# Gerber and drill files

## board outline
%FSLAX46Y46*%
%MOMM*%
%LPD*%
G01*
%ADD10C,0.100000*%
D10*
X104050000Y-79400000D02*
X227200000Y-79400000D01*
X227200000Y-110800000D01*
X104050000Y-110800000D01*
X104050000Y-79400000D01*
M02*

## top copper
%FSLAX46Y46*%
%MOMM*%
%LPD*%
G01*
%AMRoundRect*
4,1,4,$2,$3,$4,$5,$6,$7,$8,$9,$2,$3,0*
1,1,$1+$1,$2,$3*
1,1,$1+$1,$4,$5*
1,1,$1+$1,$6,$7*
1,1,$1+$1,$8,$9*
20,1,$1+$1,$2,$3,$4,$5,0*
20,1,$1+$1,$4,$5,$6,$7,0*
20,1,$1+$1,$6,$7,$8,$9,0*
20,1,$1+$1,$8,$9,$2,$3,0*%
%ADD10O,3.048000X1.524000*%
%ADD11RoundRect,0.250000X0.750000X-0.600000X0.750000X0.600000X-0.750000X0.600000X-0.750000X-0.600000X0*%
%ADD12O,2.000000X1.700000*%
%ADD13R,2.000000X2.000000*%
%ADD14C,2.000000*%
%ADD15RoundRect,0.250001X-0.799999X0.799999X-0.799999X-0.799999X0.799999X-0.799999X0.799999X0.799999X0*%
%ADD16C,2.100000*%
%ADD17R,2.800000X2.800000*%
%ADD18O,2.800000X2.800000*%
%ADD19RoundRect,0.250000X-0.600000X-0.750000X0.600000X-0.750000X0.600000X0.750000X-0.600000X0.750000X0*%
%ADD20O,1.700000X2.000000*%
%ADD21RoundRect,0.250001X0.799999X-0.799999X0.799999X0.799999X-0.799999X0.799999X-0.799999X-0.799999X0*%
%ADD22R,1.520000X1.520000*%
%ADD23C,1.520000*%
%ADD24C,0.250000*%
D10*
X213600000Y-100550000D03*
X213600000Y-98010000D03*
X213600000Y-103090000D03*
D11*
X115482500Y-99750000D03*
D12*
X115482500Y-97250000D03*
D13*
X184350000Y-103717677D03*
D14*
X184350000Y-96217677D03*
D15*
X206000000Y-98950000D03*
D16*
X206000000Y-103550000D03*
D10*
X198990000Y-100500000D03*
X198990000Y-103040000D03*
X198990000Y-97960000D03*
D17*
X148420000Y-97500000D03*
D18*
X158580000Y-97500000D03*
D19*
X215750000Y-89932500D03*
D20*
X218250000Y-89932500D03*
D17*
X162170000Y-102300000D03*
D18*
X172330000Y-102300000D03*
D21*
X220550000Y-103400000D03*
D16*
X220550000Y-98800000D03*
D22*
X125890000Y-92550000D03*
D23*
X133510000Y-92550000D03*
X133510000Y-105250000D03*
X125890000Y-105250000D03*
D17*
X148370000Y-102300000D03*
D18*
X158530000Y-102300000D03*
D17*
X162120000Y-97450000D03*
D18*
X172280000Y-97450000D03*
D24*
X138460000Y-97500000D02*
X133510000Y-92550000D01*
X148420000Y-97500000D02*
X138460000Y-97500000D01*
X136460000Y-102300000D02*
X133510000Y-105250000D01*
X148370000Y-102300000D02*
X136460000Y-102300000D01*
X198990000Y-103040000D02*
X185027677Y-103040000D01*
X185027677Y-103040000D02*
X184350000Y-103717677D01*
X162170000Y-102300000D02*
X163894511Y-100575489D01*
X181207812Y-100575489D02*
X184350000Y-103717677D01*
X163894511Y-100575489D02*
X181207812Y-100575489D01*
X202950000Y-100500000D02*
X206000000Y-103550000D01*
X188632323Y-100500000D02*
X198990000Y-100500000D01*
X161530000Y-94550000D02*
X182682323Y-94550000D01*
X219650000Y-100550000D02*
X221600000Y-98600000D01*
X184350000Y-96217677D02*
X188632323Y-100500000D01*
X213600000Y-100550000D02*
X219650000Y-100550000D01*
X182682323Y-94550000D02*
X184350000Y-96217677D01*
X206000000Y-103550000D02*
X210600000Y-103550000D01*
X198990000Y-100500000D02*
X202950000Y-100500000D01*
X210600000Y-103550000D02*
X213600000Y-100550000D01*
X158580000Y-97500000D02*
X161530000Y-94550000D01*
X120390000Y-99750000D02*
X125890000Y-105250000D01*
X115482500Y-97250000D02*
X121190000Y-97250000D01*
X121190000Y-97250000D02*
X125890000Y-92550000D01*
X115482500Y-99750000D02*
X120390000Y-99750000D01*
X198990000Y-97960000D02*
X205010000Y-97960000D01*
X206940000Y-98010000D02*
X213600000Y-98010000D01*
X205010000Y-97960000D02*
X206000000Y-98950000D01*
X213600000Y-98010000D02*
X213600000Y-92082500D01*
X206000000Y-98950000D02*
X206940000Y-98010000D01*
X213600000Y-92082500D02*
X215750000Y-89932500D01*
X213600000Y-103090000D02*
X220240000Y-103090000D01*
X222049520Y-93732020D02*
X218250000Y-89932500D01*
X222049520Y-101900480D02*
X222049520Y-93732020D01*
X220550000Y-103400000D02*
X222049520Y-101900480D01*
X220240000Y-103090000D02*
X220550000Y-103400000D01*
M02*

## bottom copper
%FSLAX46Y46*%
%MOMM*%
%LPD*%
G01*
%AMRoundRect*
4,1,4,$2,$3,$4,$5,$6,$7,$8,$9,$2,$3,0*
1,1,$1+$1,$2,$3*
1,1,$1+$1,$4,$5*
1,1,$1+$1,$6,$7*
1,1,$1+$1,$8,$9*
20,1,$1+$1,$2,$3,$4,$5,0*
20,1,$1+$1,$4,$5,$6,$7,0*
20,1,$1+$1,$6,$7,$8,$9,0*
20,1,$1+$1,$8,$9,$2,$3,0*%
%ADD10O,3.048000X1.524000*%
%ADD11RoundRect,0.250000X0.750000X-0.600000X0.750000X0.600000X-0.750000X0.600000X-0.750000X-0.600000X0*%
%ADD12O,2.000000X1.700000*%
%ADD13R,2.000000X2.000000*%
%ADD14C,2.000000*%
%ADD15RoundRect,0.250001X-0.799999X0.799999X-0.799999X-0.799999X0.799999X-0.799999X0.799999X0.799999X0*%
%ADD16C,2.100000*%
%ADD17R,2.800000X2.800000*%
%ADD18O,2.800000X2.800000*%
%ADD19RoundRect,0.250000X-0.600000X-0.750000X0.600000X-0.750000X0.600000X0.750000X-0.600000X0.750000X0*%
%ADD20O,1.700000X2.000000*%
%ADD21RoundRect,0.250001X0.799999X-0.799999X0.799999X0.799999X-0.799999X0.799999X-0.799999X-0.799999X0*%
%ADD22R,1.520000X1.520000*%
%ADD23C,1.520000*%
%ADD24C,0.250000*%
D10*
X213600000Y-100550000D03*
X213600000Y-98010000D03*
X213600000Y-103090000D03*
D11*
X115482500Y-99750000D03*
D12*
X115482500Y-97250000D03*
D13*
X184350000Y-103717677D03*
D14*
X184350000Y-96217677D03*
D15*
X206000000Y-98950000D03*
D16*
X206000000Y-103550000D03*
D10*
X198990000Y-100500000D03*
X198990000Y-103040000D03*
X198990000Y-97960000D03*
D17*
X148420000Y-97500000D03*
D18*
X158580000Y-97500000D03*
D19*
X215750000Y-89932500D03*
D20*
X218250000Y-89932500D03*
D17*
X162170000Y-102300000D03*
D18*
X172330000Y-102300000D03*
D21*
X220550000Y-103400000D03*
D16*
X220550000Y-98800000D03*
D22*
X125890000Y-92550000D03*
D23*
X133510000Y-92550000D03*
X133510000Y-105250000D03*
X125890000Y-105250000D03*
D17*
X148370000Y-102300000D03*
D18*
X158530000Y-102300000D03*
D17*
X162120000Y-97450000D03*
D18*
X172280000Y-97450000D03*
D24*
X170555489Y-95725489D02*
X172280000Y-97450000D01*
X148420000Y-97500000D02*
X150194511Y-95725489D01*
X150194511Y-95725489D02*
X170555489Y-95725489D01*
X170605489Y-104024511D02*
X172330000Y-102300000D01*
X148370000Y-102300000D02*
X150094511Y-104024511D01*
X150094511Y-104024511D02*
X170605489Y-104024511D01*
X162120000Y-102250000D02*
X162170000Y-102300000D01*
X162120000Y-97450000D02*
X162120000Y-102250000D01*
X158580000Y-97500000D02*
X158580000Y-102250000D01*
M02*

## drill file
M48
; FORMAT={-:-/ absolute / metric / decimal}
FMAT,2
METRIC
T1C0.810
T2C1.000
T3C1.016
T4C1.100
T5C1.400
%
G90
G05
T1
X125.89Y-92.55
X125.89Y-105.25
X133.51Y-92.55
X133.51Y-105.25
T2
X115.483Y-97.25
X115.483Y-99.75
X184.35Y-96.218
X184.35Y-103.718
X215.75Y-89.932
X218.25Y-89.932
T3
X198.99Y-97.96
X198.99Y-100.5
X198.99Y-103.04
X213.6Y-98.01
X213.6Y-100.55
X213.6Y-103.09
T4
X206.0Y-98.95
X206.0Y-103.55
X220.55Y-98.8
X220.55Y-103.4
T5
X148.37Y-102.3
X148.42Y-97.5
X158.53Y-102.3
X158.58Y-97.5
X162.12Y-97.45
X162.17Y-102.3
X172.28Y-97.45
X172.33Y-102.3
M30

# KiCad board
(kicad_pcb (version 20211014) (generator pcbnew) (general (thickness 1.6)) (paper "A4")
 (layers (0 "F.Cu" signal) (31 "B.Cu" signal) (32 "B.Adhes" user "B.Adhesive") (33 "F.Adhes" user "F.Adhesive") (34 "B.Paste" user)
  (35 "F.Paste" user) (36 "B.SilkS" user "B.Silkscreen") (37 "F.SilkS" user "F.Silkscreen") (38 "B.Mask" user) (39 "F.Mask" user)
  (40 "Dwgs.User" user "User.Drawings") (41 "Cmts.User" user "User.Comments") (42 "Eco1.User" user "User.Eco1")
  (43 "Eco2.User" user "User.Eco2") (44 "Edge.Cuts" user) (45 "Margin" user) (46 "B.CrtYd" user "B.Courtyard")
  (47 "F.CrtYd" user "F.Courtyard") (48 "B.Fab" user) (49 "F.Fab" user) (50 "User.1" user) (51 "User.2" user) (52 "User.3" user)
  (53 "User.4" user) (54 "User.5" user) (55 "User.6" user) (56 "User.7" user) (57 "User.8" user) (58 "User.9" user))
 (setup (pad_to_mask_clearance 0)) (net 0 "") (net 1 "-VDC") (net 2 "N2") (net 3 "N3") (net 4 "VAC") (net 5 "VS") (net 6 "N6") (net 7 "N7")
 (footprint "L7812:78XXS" (layer "F.Cu") (at 216.14 100.55 -90)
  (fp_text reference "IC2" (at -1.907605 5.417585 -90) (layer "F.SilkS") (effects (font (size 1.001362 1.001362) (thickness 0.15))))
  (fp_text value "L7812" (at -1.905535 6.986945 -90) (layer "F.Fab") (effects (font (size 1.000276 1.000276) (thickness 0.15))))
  (pad "GND" thru_hole oval locked (at 0 2.54 270) (size 1.524 3.048) (drill 1.016) (layers *.Cu *.Mask) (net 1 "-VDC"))
  (pad "IN" thru_hole oval locked (at -2.54 2.54 270) (size 1.524 3.048) (drill 1.016) (layers *.Cu *.Mask) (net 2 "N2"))
  (pad "OUT" thru_hole oval locked (at 2.54 2.54 270) (size 1.524 3.048) (drill 1.016) (layers *.Cu *.Mask) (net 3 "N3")))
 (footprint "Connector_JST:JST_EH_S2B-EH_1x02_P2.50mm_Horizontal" (layer "F.Cu") (at 115.4825 99.75 90)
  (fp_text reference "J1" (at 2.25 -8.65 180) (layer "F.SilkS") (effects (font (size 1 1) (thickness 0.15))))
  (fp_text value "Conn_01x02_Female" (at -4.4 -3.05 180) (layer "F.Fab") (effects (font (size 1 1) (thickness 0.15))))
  (pad "1" thru_hole roundrect (at 0 0 90) (size 1.7 2) (drill 1) (layers *.Cu *.Mask) (roundrect_rratio 0.147059) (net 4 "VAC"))
  (pad "2" thru_hole oval (at 2.5 0 90) (size 1.7 2) (drill 1) (layers *.Cu *.Mask) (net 4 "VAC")))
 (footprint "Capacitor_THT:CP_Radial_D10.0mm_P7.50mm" (layer "F.Cu") (at 184.35 103.717677 90)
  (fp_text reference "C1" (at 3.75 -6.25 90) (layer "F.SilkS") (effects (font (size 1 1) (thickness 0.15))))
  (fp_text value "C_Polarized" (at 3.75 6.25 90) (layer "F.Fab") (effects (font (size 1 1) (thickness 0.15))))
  (pad "1" thru_hole rect (at 0 0 90) (size 2 2) (drill 1) (layers *.Cu *.Mask) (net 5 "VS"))
  (pad "2" thru_hole circle (at 7.5 0 90) (size 2 2) (drill 1) (layers *.Cu *.Mask) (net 1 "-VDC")))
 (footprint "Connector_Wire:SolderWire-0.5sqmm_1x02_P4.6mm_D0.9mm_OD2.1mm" (layer "F.Cu") (at 206 98.95 -90)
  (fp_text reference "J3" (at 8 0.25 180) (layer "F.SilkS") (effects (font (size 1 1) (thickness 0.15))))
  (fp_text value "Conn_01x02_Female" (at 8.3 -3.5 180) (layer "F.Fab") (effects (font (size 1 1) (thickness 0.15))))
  (pad "1" thru_hole roundrect (at 0 0 270) (size 2.1 2.1) (drill 1.1) (layers *.Cu *.Mask) (roundrect_rratio 0.119048) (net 2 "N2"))
  (pad "2" thru_hole circle (at 4.6 0 270) (size 2.1 2.1) (drill 1.1) (layers *.Cu *.Mask) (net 1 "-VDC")))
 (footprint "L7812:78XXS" (layer "F.Cu") (at 196.45 100.5 90)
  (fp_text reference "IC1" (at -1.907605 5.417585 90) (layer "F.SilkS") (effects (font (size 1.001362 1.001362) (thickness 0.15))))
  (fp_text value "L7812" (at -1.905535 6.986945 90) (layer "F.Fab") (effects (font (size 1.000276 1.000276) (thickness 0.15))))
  (pad "GND" thru_hole oval locked (at 0 2.54 90) (size 1.524 3.048) (drill 1.016) (layers *.Cu *.Mask) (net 1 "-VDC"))
  (pad "IN" thru_hole oval locked (at -2.54 2.54 90) (size 1.524 3.048) (drill 1.016) (layers *.Cu *.Mask) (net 5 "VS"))
  (pad "OUT" thru_hole oval locked (at 2.54 2.54 90) (size 1.524 3.048) (drill 1.016) (layers *.Cu *.Mask) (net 2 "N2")))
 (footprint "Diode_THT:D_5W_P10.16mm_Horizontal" (layer "F.Cu") (at 148.42 97.5)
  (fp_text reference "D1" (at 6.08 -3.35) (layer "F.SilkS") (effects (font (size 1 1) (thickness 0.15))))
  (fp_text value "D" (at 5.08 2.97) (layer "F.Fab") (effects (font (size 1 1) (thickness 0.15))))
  (pad "1" thru_hole rect (at 0 0) (size 2.8 2.8) (drill 1.4) (layers *.Cu *.Mask) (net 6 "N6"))
  (pad "2" thru_hole oval (at 10.16 0) (size 2.8 2.8) (drill 1.4) (layers *.Cu *.Mask) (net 1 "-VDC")))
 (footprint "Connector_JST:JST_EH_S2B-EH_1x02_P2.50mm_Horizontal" (layer "F.Cu") (at 215.75 89.9325)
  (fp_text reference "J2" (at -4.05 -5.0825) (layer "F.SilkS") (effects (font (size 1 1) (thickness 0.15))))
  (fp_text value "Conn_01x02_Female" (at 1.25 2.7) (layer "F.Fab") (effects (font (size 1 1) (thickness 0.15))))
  (pad "1" thru_hole roundrect (at 0 0) (size 1.7 2) (drill 1) (layers *.Cu *.Mask) (roundrect_rratio 0.147059) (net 2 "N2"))
  (pad "2" thru_hole oval (at 2.5 0) (size 1.7 2) (drill 1) (layers *.Cu *.Mask) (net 3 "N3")))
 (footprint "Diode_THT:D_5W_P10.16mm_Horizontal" (layer "F.Cu") (at 162.17 102.3)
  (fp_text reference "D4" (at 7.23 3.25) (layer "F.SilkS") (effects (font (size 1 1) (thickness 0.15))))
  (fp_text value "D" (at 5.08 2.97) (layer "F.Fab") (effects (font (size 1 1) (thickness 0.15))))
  (pad "1" thru_hole rect (at 0 0) (size 2.8 2.8) (drill 1.4) (layers *.Cu *.Mask) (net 5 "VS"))
  (pad "2" thru_hole oval (at 10.16 0) (size 2.8 2.8) (drill 1.4) (layers *.Cu *.Mask) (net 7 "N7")))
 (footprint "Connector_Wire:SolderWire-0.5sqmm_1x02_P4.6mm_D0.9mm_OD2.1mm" (layer "F.Cu") (at 220.55 103.4 90)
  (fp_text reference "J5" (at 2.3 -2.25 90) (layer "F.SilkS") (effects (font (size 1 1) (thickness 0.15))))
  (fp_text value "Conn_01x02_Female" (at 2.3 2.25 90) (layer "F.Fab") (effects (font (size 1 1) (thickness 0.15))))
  (pad "1" thru_hole roundrect (at 0 0 90) (size 2.1 2.1) (drill 1.1) (layers *.Cu *.Mask) (roundrect_rratio 0.119048) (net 3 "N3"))
  (pad "2" thru_hole circle (at 4.6 0 90) (size 2.1 2.1) (drill 1.1) (layers *.Cu *.Mask) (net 1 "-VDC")))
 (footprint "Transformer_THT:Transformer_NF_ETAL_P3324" (layer "F.Cu") (at 125.89 92.55 90)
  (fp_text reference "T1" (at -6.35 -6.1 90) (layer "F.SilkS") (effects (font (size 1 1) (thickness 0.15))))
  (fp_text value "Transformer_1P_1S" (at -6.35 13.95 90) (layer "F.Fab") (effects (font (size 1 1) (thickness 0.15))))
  (pad "1" thru_hole rect (at 0 0 90) (size 1.52 1.52) (drill 0.81) (layers *.Cu *.Mask) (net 4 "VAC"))
  (pad "3" thru_hole circle (at 0 7.62 90) (size 1.52 1.52) (drill 0.81) (layers *.Cu *.Mask) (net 6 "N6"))
  (pad "4" thru_hole circle (at -12.7 7.62 90) (size 1.52 1.52) (drill 0.81) (layers *.Cu *.Mask) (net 7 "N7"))
  (pad "6" thru_hole circle (at -12.7 0 90) (size 1.52 1.52) (drill 0.81) (layers *.Cu *.Mask) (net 4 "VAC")))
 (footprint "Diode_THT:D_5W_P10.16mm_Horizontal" (layer "F.Cu") (at 148.37 102.3)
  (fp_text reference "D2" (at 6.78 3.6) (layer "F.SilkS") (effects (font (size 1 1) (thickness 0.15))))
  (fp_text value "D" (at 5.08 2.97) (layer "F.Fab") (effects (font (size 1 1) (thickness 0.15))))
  (pad "1" thru_hole rect (at 0 0) (size 2.8 2.8) (drill 1.4) (layers *.Cu *.Mask) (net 7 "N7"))
  (pad "2" thru_hole oval (at 10.16 0) (size 2.8 2.8) (drill 1.4) (layers *.Cu *.Mask) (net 1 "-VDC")))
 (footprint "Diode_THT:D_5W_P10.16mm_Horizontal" (layer "F.Cu") (at 162.12 97.45)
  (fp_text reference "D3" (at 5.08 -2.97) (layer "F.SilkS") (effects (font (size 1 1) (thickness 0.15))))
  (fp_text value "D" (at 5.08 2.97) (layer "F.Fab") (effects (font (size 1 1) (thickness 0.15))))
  (pad "1" thru_hole rect (at 0 0) (size 2.8 2.8) (drill 1.4) (layers *.Cu *.Mask) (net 5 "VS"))
  (pad "2" thru_hole oval (at 10.16 0) (size 2.8 2.8) (drill 1.4) (layers *.Cu *.Mask) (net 6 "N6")))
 (gr_rect (start 104.05 79.4) (end 227.2 110.8) (layer "Edge.Cuts") (width 0.1) (fill none))
 (segment (start 138.46 97.5) (end 133.51 92.55) (width 0.25) (layer "F.Cu") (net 6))
 (segment (start 148.42 97.5) (end 138.46 97.5) (width 0.25) (layer "F.Cu") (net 6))
 (segment (start 170.555489 95.725489) (end 172.28 97.45) (width 0.25) (layer "B.Cu") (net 6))
 (segment (start 148.42 97.5) (end 150.194511 95.725489) (width 0.25) (layer "B.Cu") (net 6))
 (segment (start 150.194511 95.725489) (end 170.555489 95.725489) (width 0.25) (layer "B.Cu") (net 6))
 (segment (start 136.46 102.3) (end 133.51 105.25) (width 0.25) (layer "F.Cu") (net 7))
 (segment (start 148.37 102.3) (end 136.46 102.3) (width 0.25) (layer "F.Cu") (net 7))
 (segment (start 170.605489 104.024511) (end 172.33 102.3) (width 0.25) (layer "B.Cu") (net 7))
 (segment (start 148.37 102.3) (end 150.094511 104.024511) (width 0.25) (layer "B.Cu") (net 7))
 (segment (start 150.094511 104.024511) (end 170.605489 104.024511) (width 0.25) (layer "B.Cu") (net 7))
 (segment (start 198.99 103.04) (end 185.027677 103.04) (width 0.25) (layer "F.Cu") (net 5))
 (segment (start 185.027677 103.04) (end 184.35 103.717677) (width 0.25) (layer "F.Cu") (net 5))
 (segment (start 162.17 102.3) (end 163.894511 100.575489) (width 0.25) (layer "F.Cu") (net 5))
 (segment (start 181.207812 100.575489) (end 184.35 103.717677) (width 0.25) (layer "F.Cu") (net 5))
 (segment (start 163.894511 100.575489) (end 181.207812 100.575489) (width 0.25) (layer "F.Cu") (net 5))
 (segment (start 162.12 102.25) (end 162.17 102.3) (width 0.25) (layer "B.Cu") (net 5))
 (segment (start 162.12 97.45) (end 162.12 102.25) (width 0.25) (layer "B.Cu") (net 5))
 (segment (start 202.95 100.5) (end 206 103.55) (width 0.25) (layer "F.Cu") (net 1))
 (segment (start 188.632323 100.5) (end 198.99 100.5) (width 0.25) (layer "F.Cu") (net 1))
 (segment (start 161.53 94.55) (end 182.682323 94.55) (width 0.25) (layer "F.Cu") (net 1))
 (segment (start 219.65 100.55) (end 221.6 98.6) (width 0.25) (layer "F.Cu") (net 1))
 (segment (start 184.35 96.217677) (end 188.632323 100.5) (width 0.25) (layer "F.Cu") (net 1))
 (segment (start 213.6 100.55) (end 219.65 100.55) (width 0.25) (layer "F.Cu") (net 1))
 (segment (start 182.682323 94.55) (end 184.35 96.217677) (width 0.25) (layer "F.Cu") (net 1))
 (segment (start 206 103.55) (end 210.6 103.55) (width 0.25) (layer "F.Cu") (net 1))
 (segment (start 198.99 100.5) (end 202.95 100.5) (width 0.25) (layer "F.Cu") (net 1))
 (segment (start 210.6 103.55) (end 213.6 100.55) (width 0.25) (layer "F.Cu") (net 1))
 (segment (start 158.58 97.5) (end 161.53 94.55) (width 0.25) (layer "F.Cu") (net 1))
 (segment (start 158.58 97.5) (end 158.58 102.25) (width 0.25) (layer "B.Cu") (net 1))
 (segment (start 120.39 99.75) (end 125.89 105.25) (width 0.25) (layer "F.Cu") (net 4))
 (segment (start 115.4825 97.25) (end 121.19 97.25) (width 0.25) (layer "F.Cu") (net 4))
 (segment (start 121.19 97.25) (end 125.89 92.55) (width 0.25) (layer "F.Cu") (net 4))
 (segment (start 115.4825 99.75) (end 120.39 99.75) (width 0.25) (layer "F.Cu") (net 4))
 (segment (start 198.99 97.96) (end 205.01 97.96) (width 0.25) (layer "F.Cu") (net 2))
 (segment (start 206.94 98.01) (end 213.6 98.01) (width 0.25) (layer "F.Cu") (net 2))
 (segment (start 205.01 97.96) (end 206 98.95) (width 0.25) (layer "F.Cu") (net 2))
 (segment (start 213.6 98.01) (end 213.6 92.0825) (width 0.25) (layer "F.Cu") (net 2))
 (segment (start 206 98.95) (end 206.94 98.01) (width 0.25) (layer "F.Cu") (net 2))
 (segment (start 213.6 92.0825) (end 215.75 89.9325) (width 0.25) (layer "F.Cu") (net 2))
 (segment (start 213.6 103.09) (end 220.24 103.09) (width 0.25) (layer "F.Cu") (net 3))
 (segment (start 222.04952 93.73202) (end 218.25 89.9325) (width 0.25) (layer "F.Cu") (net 3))
 (segment (start 222.04952 101.90048) (end 222.04952 93.73202) (width 0.25) (layer "F.Cu") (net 3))
 (segment (start 220.55 103.4) (end 222.04952 101.90048) (width 0.25) (layer "F.Cu") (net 3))
 (segment (start 220.24 103.09) (end 220.55 103.4) (width 0.25) (layer "F.Cu") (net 3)))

